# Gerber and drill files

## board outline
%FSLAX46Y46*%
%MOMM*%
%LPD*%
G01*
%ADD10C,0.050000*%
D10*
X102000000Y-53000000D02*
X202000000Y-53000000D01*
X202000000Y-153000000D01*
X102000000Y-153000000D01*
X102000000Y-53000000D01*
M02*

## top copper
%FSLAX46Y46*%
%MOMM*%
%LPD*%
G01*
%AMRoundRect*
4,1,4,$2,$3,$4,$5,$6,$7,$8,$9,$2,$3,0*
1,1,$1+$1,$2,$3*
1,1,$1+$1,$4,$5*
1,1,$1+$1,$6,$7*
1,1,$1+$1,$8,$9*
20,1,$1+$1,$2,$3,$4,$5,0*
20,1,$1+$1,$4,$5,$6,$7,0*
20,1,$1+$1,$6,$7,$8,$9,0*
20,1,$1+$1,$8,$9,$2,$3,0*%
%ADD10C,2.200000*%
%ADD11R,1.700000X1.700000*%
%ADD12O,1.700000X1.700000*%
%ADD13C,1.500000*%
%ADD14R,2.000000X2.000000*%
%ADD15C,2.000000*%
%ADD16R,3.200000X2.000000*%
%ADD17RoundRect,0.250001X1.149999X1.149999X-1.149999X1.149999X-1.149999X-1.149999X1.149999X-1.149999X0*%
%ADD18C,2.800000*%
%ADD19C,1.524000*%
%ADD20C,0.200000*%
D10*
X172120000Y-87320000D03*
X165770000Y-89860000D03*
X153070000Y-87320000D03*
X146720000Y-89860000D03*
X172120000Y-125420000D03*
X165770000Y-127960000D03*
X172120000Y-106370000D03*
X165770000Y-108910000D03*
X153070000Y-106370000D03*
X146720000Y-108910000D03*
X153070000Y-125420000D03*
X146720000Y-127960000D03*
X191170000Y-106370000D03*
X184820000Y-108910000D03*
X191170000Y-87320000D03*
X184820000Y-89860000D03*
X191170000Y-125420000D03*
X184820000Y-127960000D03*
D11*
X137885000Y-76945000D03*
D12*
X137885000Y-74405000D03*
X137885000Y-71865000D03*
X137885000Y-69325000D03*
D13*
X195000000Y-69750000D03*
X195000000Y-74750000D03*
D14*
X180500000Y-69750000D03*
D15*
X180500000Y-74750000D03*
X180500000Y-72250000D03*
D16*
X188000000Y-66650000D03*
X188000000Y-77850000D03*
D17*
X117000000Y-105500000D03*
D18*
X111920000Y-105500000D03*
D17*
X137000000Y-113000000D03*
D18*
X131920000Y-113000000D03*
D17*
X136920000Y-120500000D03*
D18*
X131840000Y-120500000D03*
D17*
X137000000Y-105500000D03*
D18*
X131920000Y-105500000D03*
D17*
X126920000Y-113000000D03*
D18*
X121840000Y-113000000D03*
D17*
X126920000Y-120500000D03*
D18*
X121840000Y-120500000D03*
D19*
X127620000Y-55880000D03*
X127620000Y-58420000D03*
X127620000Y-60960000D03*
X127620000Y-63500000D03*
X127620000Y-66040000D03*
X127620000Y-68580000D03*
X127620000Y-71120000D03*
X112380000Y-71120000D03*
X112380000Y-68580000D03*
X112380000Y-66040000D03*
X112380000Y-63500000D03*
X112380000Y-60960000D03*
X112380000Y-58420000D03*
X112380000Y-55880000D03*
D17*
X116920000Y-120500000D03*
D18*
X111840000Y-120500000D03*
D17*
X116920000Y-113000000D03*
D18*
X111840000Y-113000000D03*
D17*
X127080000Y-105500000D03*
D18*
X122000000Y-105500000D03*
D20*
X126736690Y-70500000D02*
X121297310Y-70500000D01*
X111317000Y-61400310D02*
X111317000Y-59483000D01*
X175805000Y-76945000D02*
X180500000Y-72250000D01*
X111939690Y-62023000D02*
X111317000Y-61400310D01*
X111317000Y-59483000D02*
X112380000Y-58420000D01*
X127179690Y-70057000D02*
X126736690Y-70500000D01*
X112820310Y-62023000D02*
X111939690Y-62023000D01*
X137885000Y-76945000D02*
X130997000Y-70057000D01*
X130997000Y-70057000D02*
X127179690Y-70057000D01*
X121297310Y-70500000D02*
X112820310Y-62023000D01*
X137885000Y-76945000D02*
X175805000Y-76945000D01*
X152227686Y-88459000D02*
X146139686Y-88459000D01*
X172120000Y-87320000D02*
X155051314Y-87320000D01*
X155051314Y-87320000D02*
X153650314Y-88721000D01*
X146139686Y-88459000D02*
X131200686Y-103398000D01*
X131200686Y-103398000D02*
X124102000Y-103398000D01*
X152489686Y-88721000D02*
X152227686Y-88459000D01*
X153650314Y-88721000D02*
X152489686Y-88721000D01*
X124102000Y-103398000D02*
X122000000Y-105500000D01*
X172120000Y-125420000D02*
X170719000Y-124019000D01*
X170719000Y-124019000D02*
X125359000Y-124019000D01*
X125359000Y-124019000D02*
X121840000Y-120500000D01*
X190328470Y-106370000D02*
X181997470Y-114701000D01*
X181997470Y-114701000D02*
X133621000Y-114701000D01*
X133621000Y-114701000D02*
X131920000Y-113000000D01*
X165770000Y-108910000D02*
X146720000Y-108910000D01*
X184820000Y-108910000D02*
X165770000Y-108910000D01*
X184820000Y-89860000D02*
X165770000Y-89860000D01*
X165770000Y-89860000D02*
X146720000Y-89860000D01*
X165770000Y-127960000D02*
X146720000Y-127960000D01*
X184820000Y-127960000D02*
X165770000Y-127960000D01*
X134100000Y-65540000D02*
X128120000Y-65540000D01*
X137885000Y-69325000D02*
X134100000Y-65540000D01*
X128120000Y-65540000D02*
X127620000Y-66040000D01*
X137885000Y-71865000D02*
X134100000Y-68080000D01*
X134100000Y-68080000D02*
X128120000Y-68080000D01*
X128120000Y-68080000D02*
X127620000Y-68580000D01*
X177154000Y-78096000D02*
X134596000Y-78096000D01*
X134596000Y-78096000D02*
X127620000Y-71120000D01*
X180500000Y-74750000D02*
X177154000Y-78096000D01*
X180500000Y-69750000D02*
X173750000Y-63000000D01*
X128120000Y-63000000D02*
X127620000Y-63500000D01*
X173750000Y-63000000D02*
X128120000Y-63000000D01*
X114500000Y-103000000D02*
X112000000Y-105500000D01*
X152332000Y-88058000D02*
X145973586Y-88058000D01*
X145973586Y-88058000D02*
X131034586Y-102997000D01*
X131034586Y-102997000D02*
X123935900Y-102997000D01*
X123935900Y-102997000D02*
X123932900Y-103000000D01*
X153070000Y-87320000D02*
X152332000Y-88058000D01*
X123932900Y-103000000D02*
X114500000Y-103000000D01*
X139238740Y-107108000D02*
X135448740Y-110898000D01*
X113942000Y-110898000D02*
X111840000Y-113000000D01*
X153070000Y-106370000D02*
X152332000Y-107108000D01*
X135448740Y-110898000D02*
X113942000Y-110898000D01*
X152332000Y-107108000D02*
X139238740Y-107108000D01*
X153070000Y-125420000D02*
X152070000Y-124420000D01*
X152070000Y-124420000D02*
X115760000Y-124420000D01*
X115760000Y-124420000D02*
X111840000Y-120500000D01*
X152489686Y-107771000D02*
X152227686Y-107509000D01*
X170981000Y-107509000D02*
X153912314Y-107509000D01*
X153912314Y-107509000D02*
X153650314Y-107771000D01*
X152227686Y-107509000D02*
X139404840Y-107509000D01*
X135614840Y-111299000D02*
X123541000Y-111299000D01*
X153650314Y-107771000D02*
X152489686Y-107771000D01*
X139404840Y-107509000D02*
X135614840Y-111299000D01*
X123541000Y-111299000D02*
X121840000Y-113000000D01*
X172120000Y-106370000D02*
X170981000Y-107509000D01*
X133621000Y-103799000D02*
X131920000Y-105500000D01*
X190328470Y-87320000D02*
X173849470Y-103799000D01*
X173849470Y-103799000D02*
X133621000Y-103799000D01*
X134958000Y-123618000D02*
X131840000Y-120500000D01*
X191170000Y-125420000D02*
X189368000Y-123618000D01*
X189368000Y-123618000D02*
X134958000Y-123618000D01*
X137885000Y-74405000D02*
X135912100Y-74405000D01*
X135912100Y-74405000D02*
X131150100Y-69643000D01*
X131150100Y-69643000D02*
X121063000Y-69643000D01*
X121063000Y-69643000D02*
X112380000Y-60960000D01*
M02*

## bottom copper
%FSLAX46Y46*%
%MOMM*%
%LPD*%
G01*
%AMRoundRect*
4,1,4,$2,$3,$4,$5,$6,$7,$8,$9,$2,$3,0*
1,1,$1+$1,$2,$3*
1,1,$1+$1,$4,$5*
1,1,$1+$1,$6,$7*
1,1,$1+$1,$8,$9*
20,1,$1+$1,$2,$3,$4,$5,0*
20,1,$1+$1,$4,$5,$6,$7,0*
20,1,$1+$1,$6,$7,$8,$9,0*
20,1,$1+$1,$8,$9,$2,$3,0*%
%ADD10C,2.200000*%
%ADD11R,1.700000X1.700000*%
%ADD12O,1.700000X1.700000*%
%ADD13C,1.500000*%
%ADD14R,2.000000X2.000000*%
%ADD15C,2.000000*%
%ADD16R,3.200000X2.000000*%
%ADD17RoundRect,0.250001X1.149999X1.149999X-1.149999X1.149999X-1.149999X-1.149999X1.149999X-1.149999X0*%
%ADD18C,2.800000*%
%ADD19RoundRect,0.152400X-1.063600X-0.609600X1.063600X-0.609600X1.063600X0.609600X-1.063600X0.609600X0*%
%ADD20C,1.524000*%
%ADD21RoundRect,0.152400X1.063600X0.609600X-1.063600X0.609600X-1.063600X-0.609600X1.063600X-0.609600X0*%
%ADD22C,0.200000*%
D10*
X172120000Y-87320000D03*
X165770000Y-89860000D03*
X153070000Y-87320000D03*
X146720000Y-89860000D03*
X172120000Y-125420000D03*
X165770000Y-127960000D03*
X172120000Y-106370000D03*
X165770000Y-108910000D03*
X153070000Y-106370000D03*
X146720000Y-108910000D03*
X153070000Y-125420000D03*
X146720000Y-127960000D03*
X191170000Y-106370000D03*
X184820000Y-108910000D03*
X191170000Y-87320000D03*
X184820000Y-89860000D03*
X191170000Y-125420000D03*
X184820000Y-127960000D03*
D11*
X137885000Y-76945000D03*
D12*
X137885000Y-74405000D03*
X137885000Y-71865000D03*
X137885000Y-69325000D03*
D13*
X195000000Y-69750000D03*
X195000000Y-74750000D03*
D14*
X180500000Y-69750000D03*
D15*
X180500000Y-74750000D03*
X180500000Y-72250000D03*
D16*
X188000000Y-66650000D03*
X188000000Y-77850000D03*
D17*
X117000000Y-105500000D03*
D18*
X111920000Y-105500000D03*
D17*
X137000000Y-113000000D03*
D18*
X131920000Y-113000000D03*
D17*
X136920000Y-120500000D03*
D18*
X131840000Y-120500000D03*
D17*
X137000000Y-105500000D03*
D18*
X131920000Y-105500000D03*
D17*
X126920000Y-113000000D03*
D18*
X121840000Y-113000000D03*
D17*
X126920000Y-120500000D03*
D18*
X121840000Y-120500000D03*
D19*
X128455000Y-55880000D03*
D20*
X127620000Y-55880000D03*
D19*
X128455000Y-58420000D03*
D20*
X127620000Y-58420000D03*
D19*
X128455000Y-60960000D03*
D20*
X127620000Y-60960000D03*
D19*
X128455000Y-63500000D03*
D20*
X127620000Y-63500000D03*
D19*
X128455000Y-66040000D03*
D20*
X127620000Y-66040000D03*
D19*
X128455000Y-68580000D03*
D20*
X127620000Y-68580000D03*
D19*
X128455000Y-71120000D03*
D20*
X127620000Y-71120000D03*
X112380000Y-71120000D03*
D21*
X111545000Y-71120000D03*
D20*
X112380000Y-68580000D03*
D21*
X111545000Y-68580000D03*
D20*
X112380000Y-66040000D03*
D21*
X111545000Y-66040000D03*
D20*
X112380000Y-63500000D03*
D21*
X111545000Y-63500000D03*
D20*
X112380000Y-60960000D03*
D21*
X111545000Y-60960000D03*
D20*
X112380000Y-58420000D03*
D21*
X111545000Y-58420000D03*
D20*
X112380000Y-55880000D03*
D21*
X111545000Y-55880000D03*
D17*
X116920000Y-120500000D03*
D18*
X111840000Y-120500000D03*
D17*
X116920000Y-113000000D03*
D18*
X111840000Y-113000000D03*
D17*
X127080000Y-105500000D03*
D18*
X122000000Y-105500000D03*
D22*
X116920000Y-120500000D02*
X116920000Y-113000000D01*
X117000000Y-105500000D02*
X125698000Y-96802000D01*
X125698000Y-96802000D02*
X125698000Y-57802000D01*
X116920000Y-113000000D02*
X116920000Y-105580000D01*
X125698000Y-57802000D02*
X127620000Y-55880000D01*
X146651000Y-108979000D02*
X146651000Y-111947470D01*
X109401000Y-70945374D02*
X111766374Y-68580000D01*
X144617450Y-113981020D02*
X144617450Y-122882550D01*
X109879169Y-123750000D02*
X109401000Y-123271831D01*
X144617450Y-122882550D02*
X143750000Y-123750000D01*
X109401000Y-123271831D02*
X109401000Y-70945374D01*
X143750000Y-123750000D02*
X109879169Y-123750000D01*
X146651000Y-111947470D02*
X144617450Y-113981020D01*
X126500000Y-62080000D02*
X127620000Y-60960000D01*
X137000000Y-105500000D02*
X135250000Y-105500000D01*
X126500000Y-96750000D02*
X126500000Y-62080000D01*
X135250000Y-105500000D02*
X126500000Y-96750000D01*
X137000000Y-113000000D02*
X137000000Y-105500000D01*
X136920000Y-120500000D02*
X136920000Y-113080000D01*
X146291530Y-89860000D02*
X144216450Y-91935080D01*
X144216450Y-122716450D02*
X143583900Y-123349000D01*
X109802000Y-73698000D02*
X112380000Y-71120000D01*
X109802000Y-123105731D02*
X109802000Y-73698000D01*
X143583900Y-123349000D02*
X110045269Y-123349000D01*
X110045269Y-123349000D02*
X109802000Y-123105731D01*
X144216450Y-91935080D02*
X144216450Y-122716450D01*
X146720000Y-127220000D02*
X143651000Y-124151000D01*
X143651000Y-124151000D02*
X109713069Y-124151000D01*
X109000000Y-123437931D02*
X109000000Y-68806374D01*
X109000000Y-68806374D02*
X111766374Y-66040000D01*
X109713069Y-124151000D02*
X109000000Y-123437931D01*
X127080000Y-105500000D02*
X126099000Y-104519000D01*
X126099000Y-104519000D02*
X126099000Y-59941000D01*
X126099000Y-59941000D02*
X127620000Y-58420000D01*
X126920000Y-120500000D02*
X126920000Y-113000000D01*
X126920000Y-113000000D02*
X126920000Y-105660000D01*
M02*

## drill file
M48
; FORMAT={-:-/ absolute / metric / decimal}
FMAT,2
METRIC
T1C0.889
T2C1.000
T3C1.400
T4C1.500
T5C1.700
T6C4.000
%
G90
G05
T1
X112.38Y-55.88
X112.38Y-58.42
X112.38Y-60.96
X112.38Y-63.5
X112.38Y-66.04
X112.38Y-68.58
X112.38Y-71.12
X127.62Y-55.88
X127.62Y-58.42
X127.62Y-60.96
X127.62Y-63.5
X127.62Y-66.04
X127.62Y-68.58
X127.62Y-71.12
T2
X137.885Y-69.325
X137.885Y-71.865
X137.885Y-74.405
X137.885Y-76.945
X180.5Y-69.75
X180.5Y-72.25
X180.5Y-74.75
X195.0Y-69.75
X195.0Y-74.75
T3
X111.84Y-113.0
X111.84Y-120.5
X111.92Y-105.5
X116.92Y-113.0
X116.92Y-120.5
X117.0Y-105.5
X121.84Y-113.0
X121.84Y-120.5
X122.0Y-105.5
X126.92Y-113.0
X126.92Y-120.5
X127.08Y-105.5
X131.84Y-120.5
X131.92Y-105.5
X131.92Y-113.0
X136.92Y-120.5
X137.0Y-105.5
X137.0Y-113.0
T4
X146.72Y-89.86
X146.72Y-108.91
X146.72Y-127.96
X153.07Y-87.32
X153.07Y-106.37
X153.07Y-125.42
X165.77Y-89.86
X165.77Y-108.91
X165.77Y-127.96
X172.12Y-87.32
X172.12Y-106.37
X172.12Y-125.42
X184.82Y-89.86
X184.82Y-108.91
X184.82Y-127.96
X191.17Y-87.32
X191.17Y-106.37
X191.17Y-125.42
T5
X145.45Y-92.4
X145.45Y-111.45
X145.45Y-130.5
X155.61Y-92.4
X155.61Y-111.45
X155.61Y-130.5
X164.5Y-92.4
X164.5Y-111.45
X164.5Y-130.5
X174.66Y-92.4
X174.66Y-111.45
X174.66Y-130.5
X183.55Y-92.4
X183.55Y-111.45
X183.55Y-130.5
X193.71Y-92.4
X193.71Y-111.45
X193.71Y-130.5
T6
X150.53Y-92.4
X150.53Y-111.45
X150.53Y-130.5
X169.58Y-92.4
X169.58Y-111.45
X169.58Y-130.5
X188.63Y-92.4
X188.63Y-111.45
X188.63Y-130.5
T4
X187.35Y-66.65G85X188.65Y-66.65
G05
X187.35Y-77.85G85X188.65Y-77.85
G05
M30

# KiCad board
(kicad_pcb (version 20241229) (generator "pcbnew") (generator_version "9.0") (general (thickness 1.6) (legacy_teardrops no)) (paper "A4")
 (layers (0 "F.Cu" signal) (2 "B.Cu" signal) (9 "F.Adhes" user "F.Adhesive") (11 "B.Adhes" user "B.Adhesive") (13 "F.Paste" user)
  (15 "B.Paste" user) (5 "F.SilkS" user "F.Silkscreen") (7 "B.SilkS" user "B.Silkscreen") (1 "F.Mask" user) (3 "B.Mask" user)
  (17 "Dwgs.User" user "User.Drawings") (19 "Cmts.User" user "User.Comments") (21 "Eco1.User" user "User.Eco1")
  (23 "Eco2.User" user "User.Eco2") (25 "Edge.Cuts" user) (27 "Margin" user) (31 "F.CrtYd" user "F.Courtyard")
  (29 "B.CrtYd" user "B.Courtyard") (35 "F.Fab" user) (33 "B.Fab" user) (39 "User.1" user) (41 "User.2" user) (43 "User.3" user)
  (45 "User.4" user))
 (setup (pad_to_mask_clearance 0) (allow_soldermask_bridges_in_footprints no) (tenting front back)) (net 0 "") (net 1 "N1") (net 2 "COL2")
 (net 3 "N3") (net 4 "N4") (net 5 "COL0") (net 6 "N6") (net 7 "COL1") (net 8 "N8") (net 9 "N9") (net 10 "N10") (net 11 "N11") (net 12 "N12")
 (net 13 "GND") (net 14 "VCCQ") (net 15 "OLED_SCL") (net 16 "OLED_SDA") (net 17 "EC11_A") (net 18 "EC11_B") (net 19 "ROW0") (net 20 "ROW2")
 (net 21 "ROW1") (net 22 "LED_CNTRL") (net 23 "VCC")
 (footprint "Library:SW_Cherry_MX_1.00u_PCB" (layer "F.Cu") (at 172.12 87.32)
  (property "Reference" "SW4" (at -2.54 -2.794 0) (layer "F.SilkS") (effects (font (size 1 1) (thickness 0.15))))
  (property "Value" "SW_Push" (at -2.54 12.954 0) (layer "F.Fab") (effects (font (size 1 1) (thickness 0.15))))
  (pad "" np_thru_hole circle (at -7.62 5.08) (size 1.7 1.7) (drill 1.7) (layers "*.Cu" "*.Mask"))
  (pad "" np_thru_hole circle (at -2.54 5.08) (size 4 4) (drill 4) (layers "*.Cu" "*.Mask"))
  (pad "" np_thru_hole circle (at 2.54 5.08) (size 1.7 1.7) (drill 1.7) (layers "*.Cu" "*.Mask"))
  (pad "1" thru_hole circle (at 0 0) (size 2.2 2.2) (drill 1.5) (layers "*.Cu" "*.Mask") (remove_unused_layers no) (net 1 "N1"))
  (pad "2" thru_hole circle (at -6.35 2.54) (size 2.2 2.2) (drill 1.5) (layers "*.Cu" "*.Mask") (remove_unused_layers no) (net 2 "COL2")))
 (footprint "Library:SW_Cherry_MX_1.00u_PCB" (layer "F.Cu") (at 153.07 87.32)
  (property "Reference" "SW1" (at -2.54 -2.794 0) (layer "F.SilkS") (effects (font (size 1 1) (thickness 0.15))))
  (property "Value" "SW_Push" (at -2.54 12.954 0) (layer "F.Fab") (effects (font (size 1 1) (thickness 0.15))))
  (pad "" np_thru_hole circle (at -7.62 5.08) (size 1.7 1.7) (drill 1.7) (layers "*.Cu" "*.Mask"))
  (pad "" np_thru_hole circle (at -2.54 5.08) (size 4 4) (drill 4) (layers "*.Cu" "*.Mask"))
  (pad "" np_thru_hole circle (at 2.54 5.08) (size 1.7 1.7) (drill 1.7) (layers "*.Cu" "*.Mask"))
  (pad "1" thru_hole circle (at 0 0) (size 2.2 2.2) (drill 1.5) (layers "*.Cu" "*.Mask") (remove_unused_layers no) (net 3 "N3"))
  (pad "2" thru_hole circle (at -6.35 2.54) (size 2.2 2.2) (drill 1.5) (layers "*.Cu" "*.Mask") (remove_unused_layers no) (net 2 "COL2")))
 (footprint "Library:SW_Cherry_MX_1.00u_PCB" (layer "F.Cu") (at 172.12 125.42)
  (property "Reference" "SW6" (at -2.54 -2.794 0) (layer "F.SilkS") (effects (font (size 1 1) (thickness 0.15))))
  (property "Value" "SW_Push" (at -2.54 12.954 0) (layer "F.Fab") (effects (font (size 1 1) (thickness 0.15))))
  (pad "" np_thru_hole circle (at -7.62 5.08) (size 1.7 1.7) (drill 1.7) (layers "*.Cu" "*.Mask"))
  (pad "" np_thru_hole circle (at -2.54 5.08) (size 4 4) (drill 4) (layers "*.Cu" "*.Mask"))
  (pad "" np_thru_hole circle (at 2.54 5.08) (size 1.7 1.7) (drill 1.7) (layers "*.Cu" "*.Mask"))
  (pad "1" thru_hole circle (at 0 0) (size 2.2 2.2) (drill 1.5) (layers "*.Cu" "*.Mask") (remove_unused_layers no) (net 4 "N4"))
  (pad "2" thru_hole circle (at -6.35 2.54) (size 2.2 2.2) (drill 1.5) (layers "*.Cu" "*.Mask") (remove_unused_layers no) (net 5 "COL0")))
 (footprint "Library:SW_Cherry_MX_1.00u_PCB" (layer "F.Cu") (at 172.12 106.37)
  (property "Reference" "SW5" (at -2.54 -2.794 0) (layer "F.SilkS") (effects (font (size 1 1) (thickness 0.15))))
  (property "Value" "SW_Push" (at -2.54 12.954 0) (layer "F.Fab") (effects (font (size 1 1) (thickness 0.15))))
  (pad "" np_thru_hole circle (at -7.62 5.08) (size 1.7 1.7) (drill 1.7) (layers "*.Cu" "*.Mask"))
  (pad "" np_thru_hole circle (at -2.54 5.08) (size 4 4) (drill 4) (layers "*.Cu" "*.Mask"))
  (pad "" np_thru_hole circle (at 2.54 5.08) (size 1.7 1.7) (drill 1.7) (layers "*.Cu" "*.Mask"))
  (pad "1" thru_hole circle (at 0 0) (size 2.2 2.2) (drill 1.5) (layers "*.Cu" "*.Mask") (remove_unused_layers no) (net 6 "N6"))
  (pad "2" thru_hole circle (at -6.35 2.54) (size 2.2 2.2) (drill 1.5) (layers "*.Cu" "*.Mask") (remove_unused_layers no) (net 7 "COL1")))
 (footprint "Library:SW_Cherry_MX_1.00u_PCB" (layer "F.Cu") (at 153.07 106.37)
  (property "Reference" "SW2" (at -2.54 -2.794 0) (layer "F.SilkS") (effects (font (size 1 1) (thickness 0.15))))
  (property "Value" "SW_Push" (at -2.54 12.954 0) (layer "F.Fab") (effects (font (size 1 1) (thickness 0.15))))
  (pad "" np_thru_hole circle (at -7.62 5.08) (size 1.7 1.7) (drill 1.7) (layers "*.Cu" "*.Mask"))
  (pad "" np_thru_hole circle (at -2.54 5.08) (size 4 4) (drill 4) (layers "*.Cu" "*.Mask"))
  (pad "" np_thru_hole circle (at 2.54 5.08) (size 1.7 1.7) (drill 1.7) (layers "*.Cu" "*.Mask"))
  (pad "1" thru_hole circle (at 0 0) (size 2.2 2.2) (drill 1.5) (layers "*.Cu" "*.Mask") (remove_unused_layers no) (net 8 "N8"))
  (pad "2" thru_hole circle (at -6.35 2.54) (size 2.2 2.2) (drill 1.5) (layers "*.Cu" "*.Mask") (remove_unused_layers no) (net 7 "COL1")))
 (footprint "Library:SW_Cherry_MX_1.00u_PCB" (layer "F.Cu") (at 153.07 125.42)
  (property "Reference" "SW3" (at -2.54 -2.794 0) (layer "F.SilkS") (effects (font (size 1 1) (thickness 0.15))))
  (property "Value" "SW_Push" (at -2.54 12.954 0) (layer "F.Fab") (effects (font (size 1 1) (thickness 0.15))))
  (pad "" np_thru_hole circle (at -7.62 5.08) (size 1.7 1.7) (drill 1.7) (layers "*.Cu" "*.Mask"))
  (pad "" np_thru_hole circle (at -2.54 5.08) (size 4 4) (drill 4) (layers "*.Cu" "*.Mask"))
  (pad "" np_thru_hole circle (at 2.54 5.08) (size 1.7 1.7) (drill 1.7) (layers "*.Cu" "*.Mask"))
  (pad "1" thru_hole circle (at 0 0) (size 2.2 2.2) (drill 1.5) (layers "*.Cu" "*.Mask") (remove_unused_layers no) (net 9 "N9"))
  (pad "2" thru_hole circle (at -6.35 2.54) (size 2.2 2.2) (drill 1.5) (layers "*.Cu" "*.Mask") (remove_unused_layers no) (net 5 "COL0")))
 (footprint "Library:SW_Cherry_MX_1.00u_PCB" (layer "F.Cu") (at 191.17 106.37)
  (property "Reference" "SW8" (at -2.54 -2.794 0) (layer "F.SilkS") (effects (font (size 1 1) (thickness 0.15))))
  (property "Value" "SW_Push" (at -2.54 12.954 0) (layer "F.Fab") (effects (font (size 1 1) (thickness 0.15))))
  (pad "" np_thru_hole circle (at -7.62 5.08) (size 1.7 1.7) (drill 1.7) (layers "*.Cu" "*.Mask"))
  (pad "" np_thru_hole circle (at -2.54 5.08) (size 4 4) (drill 4) (layers "*.Cu" "*.Mask"))
  (pad "" np_thru_hole circle (at 2.54 5.08) (size 1.7 1.7) (drill 1.7) (layers "*.Cu" "*.Mask"))
  (pad "1" thru_hole circle (at 0 0) (size 2.2 2.2) (drill 1.5) (layers "*.Cu" "*.Mask") (remove_unused_layers no) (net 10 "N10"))
  (pad "2" thru_hole circle (at -6.35 2.54) (size 2.2 2.2) (drill 1.5) (layers "*.Cu" "*.Mask") (remove_unused_layers no) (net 7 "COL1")))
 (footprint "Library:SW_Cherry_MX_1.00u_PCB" (layer "F.Cu") (at 191.17 87.32)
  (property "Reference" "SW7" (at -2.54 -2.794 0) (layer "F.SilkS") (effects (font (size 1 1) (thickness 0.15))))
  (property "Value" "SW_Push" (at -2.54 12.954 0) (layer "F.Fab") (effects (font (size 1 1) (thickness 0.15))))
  (pad "" np_thru_hole circle (at -7.62 5.08) (size 1.7 1.7) (drill 1.7) (layers "*.Cu" "*.Mask"))
  (pad "" np_thru_hole circle (at -2.54 5.08) (size 4 4) (drill 4) (layers "*.Cu" "*.Mask"))
  (pad "" np_thru_hole circle (at 2.54 5.08) (size 1.7 1.7) (drill 1.7) (layers "*.Cu" "*.Mask"))
  (pad "1" thru_hole circle (at 0 0) (size 2.2 2.2) (drill 1.5) (layers "*.Cu" "*.Mask") (remove_unused_layers no) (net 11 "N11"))
  (pad "2" thru_hole circle (at -6.35 2.54) (size 2.2 2.2) (drill 1.5) (layers "*.Cu" "*.Mask") (remove_unused_layers no) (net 2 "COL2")))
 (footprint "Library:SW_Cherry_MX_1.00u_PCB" (layer "F.Cu") (at 191.17 125.42)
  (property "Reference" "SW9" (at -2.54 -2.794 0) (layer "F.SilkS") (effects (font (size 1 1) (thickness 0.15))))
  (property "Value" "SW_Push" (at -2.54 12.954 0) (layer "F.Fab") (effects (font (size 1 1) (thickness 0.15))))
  (pad "" np_thru_hole circle (at -7.62 5.08) (size 1.7 1.7) (drill 1.7) (layers "*.Cu" "*.Mask"))
  (pad "" np_thru_hole circle (at -2.54 5.08) (size 4 4) (drill 4) (layers "*.Cu" "*.Mask"))
  (pad "" np_thru_hole circle (at 2.54 5.08) (size 1.7 1.7) (drill 1.7) (layers "*.Cu" "*.Mask"))
  (pad "1" thru_hole circle (at 0 0) (size 2.2 2.2) (drill 1.5) (layers "*.Cu" "*.Mask") (remove_unused_layers no) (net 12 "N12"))
  (pad "2" thru_hole circle (at -6.35 2.54) (size 2.2 2.2) (drill 1.5) (layers "*.Cu" "*.Mask") (remove_unused_layers no) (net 5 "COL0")))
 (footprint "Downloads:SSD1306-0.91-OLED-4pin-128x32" (layer "F.Cu") (at 174.385 79.135 180)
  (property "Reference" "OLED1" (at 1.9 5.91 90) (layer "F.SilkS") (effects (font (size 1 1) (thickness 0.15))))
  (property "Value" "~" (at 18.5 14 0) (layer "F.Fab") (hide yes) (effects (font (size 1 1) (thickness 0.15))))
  (pad "1" thru_hole rect (at 36.5 2.19 180) (size 1.7 1.7) (drill 1) (layers "*.Cu" "*.Mask") (remove_unused_layers no) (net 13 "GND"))
  (pad "2" thru_hole oval (at 36.5 4.73 180) (size 1.7 1.7) (drill 1) (layers "*.Cu" "*.Mask") (remove_unused_layers no) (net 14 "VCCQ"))
  (pad "3" thru_hole oval (at 36.5 7.27 180) (size 1.7 1.7) (drill 1) (layers "*.Cu" "*.Mask") (remove_unused_layers no) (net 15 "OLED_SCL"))
  (pad "4" thru_hole oval (at 36.5 9.81 180) (size 1.7 1.7) (drill 1) (layers "*.Cu" "*.Mask") (remove_unused_layers no) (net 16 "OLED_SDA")))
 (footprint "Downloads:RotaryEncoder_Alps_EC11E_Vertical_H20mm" (layer "F.Cu") (at 180.5 69.75)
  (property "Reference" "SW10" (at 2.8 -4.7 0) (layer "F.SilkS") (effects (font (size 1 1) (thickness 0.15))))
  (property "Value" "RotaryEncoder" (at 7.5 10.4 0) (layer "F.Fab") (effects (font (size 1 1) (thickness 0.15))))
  (pad "" thru_hole circle (at 14.5 0) (size 1.5 1.5) (drill 1) (layers "*.Cu" "*.Mask") (remove_unused_layers no))
  (pad "" thru_hole circle (at 14.5 5) (size 1.5 1.5) (drill 1) (layers "*.Cu" "*.Mask") (remove_unused_layers no))
  (pad "A" thru_hole rect (at 0 0) (size 2 2) (drill 1) (layers "*.Cu" "*.Mask") (remove_unused_layers no) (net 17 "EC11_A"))
  (pad "B" thru_hole circle (at 0 5) (size 2 2) (drill 1) (layers "*.Cu" "*.Mask") (remove_unused_layers no) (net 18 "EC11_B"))
  (pad "C" thru_hole circle (at 0 2.5) (size 2 2) (drill 1) (layers "*.Cu" "*.Mask") (remove_unused_layers no) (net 13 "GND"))
  (pad "MP" thru_hole rect (at 7.5 -3.1) (size 3.2 2) (drill oval 2.8 1.5) (layers "*.Cu" "*.Mask") (remove_unused_layers no))
  (pad "MP" thru_hole rect (at 7.5 8.1) (size 3.2 2) (drill oval 2.8 1.5) (layers "*.Cu" "*.Mask") (remove_unused_layers no)))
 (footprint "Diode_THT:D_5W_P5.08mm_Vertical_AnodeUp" (layer "B.Cu") (at 117 105.5 180)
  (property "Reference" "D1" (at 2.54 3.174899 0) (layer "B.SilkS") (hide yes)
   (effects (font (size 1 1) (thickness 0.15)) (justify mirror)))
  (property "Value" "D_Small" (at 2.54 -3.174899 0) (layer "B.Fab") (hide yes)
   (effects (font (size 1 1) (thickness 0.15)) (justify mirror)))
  (pad "1" thru_hole roundrect (at 0 0 180) (size 2.8 2.8) (drill 1.4) (layers "*.Cu" "*.Mask") (remove_unused_layers no)
   (roundrect_rratio 0.089286) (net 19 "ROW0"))
  (pad "2" thru_hole circle (at 5.08 0 180) (size 2.8 2.8) (drill 1.4) (layers "*.Cu" "*.Mask") (remove_unused_layers no) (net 3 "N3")))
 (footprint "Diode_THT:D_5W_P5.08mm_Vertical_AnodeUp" (layer "B.Cu") (at 137 113 180)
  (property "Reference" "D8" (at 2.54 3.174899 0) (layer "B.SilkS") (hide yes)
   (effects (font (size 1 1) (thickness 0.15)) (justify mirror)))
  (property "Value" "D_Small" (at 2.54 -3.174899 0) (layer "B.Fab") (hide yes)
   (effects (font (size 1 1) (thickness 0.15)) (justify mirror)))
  (pad "1" thru_hole roundrect (at 0 0 180) (size 2.8 2.8) (drill 1.4) (layers "*.Cu" "*.Mask") (remove_unused_layers no)
   (roundrect_rratio 0.089286) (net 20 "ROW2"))
  (pad "2" thru_hole circle (at 5.08 0 180) (size 2.8 2.8) (drill 1.4) (layers "*.Cu" "*.Mask") (remove_unused_layers no) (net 10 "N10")))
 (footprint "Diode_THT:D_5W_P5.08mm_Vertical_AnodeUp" (layer "B.Cu") (at 136.92 120.5 180)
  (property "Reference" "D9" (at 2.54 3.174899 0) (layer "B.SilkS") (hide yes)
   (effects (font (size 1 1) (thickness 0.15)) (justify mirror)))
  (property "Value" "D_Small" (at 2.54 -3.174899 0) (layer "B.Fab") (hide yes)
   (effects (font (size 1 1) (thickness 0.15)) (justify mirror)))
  (pad "1" thru_hole roundrect (at 0 0 180) (size 2.8 2.8) (drill 1.4) (layers "*.Cu" "*.Mask") (remove_unused_layers no)
   (roundrect_rratio 0.089286) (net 20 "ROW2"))
  (pad "2" thru_hole circle (at 5.08 0 180) (size 2.8 2.8) (drill 1.4) (layers "*.Cu" "*.Mask") (remove_unused_layers no) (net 12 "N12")))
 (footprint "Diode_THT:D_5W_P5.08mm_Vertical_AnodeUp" (layer "B.Cu") (at 137 105.5 180)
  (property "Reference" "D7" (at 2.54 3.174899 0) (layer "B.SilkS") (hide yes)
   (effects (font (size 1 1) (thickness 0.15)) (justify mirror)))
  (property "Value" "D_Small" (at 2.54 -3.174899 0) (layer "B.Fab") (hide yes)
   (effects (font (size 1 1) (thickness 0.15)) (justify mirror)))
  (pad "1" thru_hole roundrect (at 0 0 180) (size 2.8 2.8) (drill 1.4) (layers "*.Cu" "*.Mask") (remove_unused_layers no)
   (roundrect_rratio 0.089286) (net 20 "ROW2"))
  (pad "2" thru_hole circle (at 5.08 0 180) (size 2.8 2.8) (drill 1.4) (layers "*.Cu" "*.Mask") (remove_unused_layers no) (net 11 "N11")))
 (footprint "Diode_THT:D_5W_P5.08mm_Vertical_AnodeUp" (layer "B.Cu") (at 126.92 113 180)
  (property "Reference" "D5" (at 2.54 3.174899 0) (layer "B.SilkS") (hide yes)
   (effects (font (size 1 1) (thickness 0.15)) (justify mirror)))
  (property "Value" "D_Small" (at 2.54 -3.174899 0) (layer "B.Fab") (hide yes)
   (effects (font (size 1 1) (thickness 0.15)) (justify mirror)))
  (pad "1" thru_hole roundrect (at 0 0 180) (size 2.8 2.8) (drill 1.4) (layers "*.Cu" "*.Mask") (remove_unused_layers no)
   (roundrect_rratio 0.089286) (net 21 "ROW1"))
  (pad "2" thru_hole circle (at 5.08 0 180) (size 2.8 2.8) (drill 1.4) (layers "*.Cu" "*.Mask") (remove_unused_layers no) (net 6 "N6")))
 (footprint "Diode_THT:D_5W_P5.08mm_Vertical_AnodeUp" (layer "B.Cu") (at 126.92 120.5 180)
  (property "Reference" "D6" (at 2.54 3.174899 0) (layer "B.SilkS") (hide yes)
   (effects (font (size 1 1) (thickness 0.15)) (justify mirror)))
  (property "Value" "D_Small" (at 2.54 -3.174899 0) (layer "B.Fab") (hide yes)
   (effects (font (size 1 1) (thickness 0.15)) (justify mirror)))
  (pad "1" thru_hole roundrect (at 0 0 180) (size 2.8 2.8) (drill 1.4) (layers "*.Cu" "*.Mask") (remove_unused_layers no)
   (roundrect_rratio 0.089286) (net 21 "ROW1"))
  (pad "2" thru_hole circle (at 5.08 0 180) (size 2.8 2.8) (drill 1.4) (layers "*.Cu" "*.Mask") (remove_unused_layers no) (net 4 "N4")))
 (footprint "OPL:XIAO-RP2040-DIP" (layer "B.Cu") (at 120 63.5 180)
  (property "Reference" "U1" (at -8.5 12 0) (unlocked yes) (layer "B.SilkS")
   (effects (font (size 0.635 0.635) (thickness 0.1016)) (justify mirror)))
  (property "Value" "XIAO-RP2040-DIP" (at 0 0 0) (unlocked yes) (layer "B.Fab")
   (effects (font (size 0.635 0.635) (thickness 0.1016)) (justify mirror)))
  (pad "1" smd roundrect (at -8.455 7.62) (size 2.432 1.524) (layers "B.Cu" "B.Mask") (roundrect_rratio 0.1) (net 19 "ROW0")
   (thermal_bridge_angle 45))
  (pad "1" thru_hole circle (at -7.62 7.62) (size 1.524 1.524) (drill 0.889) (layers "*.Cu" "*.Mask") (remove_unused_layers no)
   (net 19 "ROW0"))
  (pad "2" smd roundrect (at -8.455 5.08) (size 2.432 1.524) (layers "B.Cu" "B.Mask") (roundrect_rratio 0.1) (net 21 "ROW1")
   (thermal_bridge_angle 45))
  (pad "2" thru_hole circle (at -7.62 5.08) (size 1.524 1.524) (drill 0.889) (layers "*.Cu" "*.Mask") (remove_unused_layers no)
   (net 21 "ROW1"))
  (pad "3" smd roundrect (at -8.455 2.54) (size 2.432 1.524) (layers "B.Cu" "B.Mask") (roundrect_rratio 0.1) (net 20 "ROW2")
   (thermal_bridge_angle 45))
  (pad "3" thru_hole circle (at -7.62 2.54) (size 1.524 1.524) (drill 0.889) (layers "*.Cu" "*.Mask") (remove_unused_layers no)
   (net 20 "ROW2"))
  (pad "4" smd roundrect (at -8.455 0) (size 2.432 1.524) (layers "B.Cu" "B.Mask") (roundrect_rratio 0.1) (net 17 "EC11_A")
   (thermal_bridge_angle 45))
  (pad "4" thru_hole circle (at -7.62 0) (size 1.524 1.524) (drill 0.889) (layers "*.Cu" "*.Mask") (remove_unused_layers no)
   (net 17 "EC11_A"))
  (pad "5" smd roundrect (at -8.455 -2.54) (size 2.432 1.524) (layers "B.Cu" "B.Mask") (roundrect_rratio 0.1) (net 16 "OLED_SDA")
   (thermal_bridge_angle 45))
  (pad "5" thru_hole circle (at -7.62 -2.54) (size 1.524 1.524) (drill 0.889) (layers "*.Cu" "*.Mask") (remove_unused_layers no)
   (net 16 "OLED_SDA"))
  (pad "6" smd roundrect (at -8.455 -5.08) (size 2.432 1.524) (layers "B.Cu" "B.Mask") (roundrect_rratio 0.1) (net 15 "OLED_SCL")
   (thermal_bridge_angle 45))
  (pad "6" thru_hole circle (at -7.62 -5.08) (size 1.524 1.524) (drill 0.889) (layers "*.Cu" "*.Mask") (remove_unused_layers no)
   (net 15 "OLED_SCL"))
  (pad "7" smd roundrect (at -8.455 -7.62) (size 2.432 1.524) (layers "B.Cu" "B.Mask") (roundrect_rratio 0.1) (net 18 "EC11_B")
   (thermal_bridge_angle 45))
  (pad "7" thru_hole circle (at -7.62 -7.62) (size 1.524 1.524) (drill 0.889) (layers "*.Cu" "*.Mask") (remove_unused_layers no)
   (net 18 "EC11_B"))
  (pad "8" thru_hole circle (at 7.62 -7.62 180) (size 1.524 1.524) (drill 0.889) (layers "*.Cu" "*.Mask") (remove_unused_layers no)
   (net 2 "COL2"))
  (pad "8" smd roundrect (at 8.455 -7.62 180) (size 2.432 1.524) (layers "B.Cu" "B.Mask") (roundrect_rratio 0.1) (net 2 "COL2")
   (thermal_bridge_angle 45))
  (pad "9" thru_hole circle (at 7.62 -5.08 180) (size 1.524 1.524) (drill 0.889) (layers "*.Cu" "*.Mask") (remove_unused_layers no)
   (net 7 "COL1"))
  (pad "9" smd roundrect (at 8.455 -5.08 180) (size 2.432 1.524) (layers "B.Cu" "B.Mask") (roundrect_rratio 0.1) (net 7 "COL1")
   (thermal_bridge_angle 45))
  (pad "10" thru_hole circle (at 7.62 -2.54 180) (size 1.524 1.524) (drill 0.889) (layers "*.Cu" "*.Mask") (remove_unused_layers no)
   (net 5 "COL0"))
  (pad "10" smd roundrect (at 8.455 -2.54 180) (size 2.432 1.524) (layers "B.Cu" "B.Mask") (roundrect_rratio 0.1) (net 5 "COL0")
   (thermal_bridge_angle 45))
  (pad "11" thru_hole circle (at 7.62 0 180) (size 1.524 1.524) (drill 0.889) (layers "*.Cu" "*.Mask") (remove_unused_layers no)
   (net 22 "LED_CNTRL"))
  (pad "11" smd roundrect (at 8.455 0 180) (size 2.432 1.524) (layers "B.Cu" "B.Mask") (roundrect_rratio 0.1) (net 22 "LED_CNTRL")
   (thermal_bridge_angle 45))
  (pad "12" thru_hole circle (at 7.62 2.54 180) (size 1.524 1.524) (drill 0.889) (layers "*.Cu" "*.Mask") (remove_unused_layers no)
   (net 14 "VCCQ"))
  (pad "12" smd roundrect (at 8.455 2.54 180) (size 2.432 1.524) (layers "B.Cu" "B.Mask") (roundrect_rratio 0.1) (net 14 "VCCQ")
   (thermal_bridge_angle 45))
  (pad "13" thru_hole circle (at 7.62 5.08 180) (size 1.524 1.524) (drill 0.889) (layers "*.Cu" "*.Mask") (remove_unused_layers no)
   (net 13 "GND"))
  (pad "13" smd roundrect (at 8.455 5.08 180) (size 2.432 1.524) (layers "B.Cu" "B.Mask") (roundrect_rratio 0.1) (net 13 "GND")
   (thermal_bridge_angle 45))
  (pad "14" thru_hole circle (at 7.62 7.62 180) (size 1.524 1.524) (drill 0.889) (layers "*.Cu" "*.Mask") (remove_unused_layers no)
   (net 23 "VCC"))
  (pad "14" smd roundrect (at 8.455 7.62 180) (size 2.432 1.524) (layers "B.Cu" "B.Mask") (roundrect_rratio 0.1) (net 23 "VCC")
   (thermal_bridge_angle 45)))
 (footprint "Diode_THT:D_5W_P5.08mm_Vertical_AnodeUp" (layer "B.Cu") (at 116.92 120.5 180)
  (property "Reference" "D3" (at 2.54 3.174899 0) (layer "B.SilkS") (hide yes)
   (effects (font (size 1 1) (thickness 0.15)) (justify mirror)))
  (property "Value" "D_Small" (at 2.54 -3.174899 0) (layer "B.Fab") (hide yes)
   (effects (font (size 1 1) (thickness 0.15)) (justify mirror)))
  (pad "1" thru_hole roundrect (at 0 0 180) (size 2.8 2.8) (drill 1.4) (layers "*.Cu" "*.Mask") (remove_unused_layers no)
   (roundrect_rratio 0.089286) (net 19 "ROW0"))
  (pad "2" thru_hole circle (at 5.08 0 180) (size 2.8 2.8) (drill 1.4) (layers "*.Cu" "*.Mask") (remove_unused_layers no) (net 9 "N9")))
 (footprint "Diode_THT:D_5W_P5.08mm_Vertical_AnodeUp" (layer "B.Cu") (at 116.92 113 180)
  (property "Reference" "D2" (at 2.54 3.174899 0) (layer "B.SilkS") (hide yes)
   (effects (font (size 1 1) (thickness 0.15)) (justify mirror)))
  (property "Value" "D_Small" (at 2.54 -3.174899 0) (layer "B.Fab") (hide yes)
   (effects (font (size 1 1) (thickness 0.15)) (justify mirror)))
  (pad "1" thru_hole roundrect (at 0 0 180) (size 2.8 2.8) (drill 1.4) (layers "*.Cu" "*.Mask") (remove_unused_layers no)
   (roundrect_rratio 0.089286) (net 19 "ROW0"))
  (pad "2" thru_hole circle (at 5.08 0 180) (size 2.8 2.8) (drill 1.4) (layers "*.Cu" "*.Mask") (remove_unused_layers no) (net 8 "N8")))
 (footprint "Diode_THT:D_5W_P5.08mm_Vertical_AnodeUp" (layer "B.Cu") (at 127.08 105.5 180)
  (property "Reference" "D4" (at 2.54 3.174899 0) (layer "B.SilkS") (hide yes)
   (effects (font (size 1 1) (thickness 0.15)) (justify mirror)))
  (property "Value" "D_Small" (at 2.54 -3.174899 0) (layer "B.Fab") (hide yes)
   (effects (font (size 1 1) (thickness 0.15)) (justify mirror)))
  (pad "1" thru_hole roundrect (at 0 0 180) (size 2.8 2.8) (drill 1.4) (layers "*.Cu" "*.Mask") (remove_unused_layers no)
   (roundrect_rratio 0.089286) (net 21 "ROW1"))
  (pad "2" thru_hole circle (at 5.08 0 180) (size 2.8 2.8) (drill 1.4) (layers "*.Cu" "*.Mask") (remove_unused_layers no) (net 1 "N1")))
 (gr_rect (start 102 53) (end 202 153) (stroke (width 0.05) (type default)) (fill no) (layer "Edge.Cuts"))
 (segment (start 126.73669 70.5) (end 121.29731 70.5) (width 0.2) (layer "F.Cu") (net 13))
 (segment (start 111.317 61.40031) (end 111.317 59.483) (width 0.2) (layer "F.Cu") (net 13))
 (segment (start 175.805 76.945) (end 180.5 72.25) (width 0.2) (layer "F.Cu") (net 13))
 (segment (start 111.93969 62.023) (end 111.317 61.40031) (width 0.2) (layer "F.Cu") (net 13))
 (segment (start 111.317 59.483) (end 112.38 58.42) (width 0.2) (layer "F.Cu") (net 13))
 (segment (start 127.17969 70.057) (end 126.73669 70.5) (width 0.2) (layer "F.Cu") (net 13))
 (segment (start 112.82031 62.023) (end 111.93969 62.023) (width 0.2) (layer "F.Cu") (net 13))
 (segment (start 137.885 76.945) (end 130.997 70.057) (width 0.2) (layer "F.Cu") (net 13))
 (segment (start 130.997 70.057) (end 127.17969 70.057) (width 0.2) (layer "F.Cu") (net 13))
 (segment (start 121.29731 70.5) (end 112.82031 62.023) (width 0.2) (layer "F.Cu") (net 13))
 (segment (start 137.885 76.945) (end 175.805 76.945) (width 0.2) (layer "F.Cu") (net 13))
 (segment (start 116.92 120.5) (end 116.92 113) (width 0.2) (layer "B.Cu") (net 19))
 (segment (start 117 105.5) (end 125.698 96.802) (width 0.2) (layer "B.Cu") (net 19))
 (segment (start 125.698 96.802) (end 125.698 57.802) (width 0.2) (layer "B.Cu") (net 19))
 (segment (start 116.92 113) (end 116.92 105.58) (width 0.2) (layer "B.Cu") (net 19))
 (segment (start 125.698 57.802) (end 127.62 55.88) (width 0.2) (layer "B.Cu") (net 19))
 (segment (start 152.227686 88.459) (end 146.139686 88.459) (width 0.2) (layer "F.Cu") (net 1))
 (segment (start 172.12 87.32) (end 155.051314 87.32) (width 0.2) (layer "F.Cu") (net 1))
 (segment (start 155.051314 87.32) (end 153.650314 88.721) (width 0.2) (layer "F.Cu") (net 1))
 (segment (start 146.139686 88.459) (end 131.200686 103.398) (width 0.2) (layer "F.Cu") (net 1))
 (segment (start 131.200686 103.398) (end 124.102 103.398) (width 0.2) (layer "F.Cu") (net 1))
 (segment (start 152.489686 88.721) (end 152.227686 88.459) (width 0.2) (layer "F.Cu") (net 1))
 (segment (start 153.650314 88.721) (end 152.489686 88.721) (width 0.2) (layer "F.Cu") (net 1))
 (segment (start 124.102 103.398) (end 122 105.5) (width 0.2) (layer "F.Cu") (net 1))
 (segment (start 172.12 125.42) (end 170.719 124.019) (width 0.2) (layer "F.Cu") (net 4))
 (segment (start 170.719 124.019) (end 125.359 124.019) (width 0.2) (layer "F.Cu") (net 4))
 (segment (start 125.359 124.019) (end 121.84 120.5) (width 0.2) (layer "F.Cu") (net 4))
 (segment (start 190.32847 106.37) (end 181.99747 114.701) (width 0.2) (layer "F.Cu") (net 10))
 (segment (start 181.99747 114.701) (end 133.621 114.701) (width 0.2) (layer "F.Cu") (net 10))
 (segment (start 133.621 114.701) (end 131.92 113) (width 0.2) (layer "F.Cu") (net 10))
 (segment (start 165.77 108.91) (end 146.72 108.91) (width 0.2) (layer "F.Cu") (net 7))
 (segment (start 184.82 108.91) (end 165.77 108.91) (width 0.2) (layer "F.Cu") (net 7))
 (segment (start 146.651 108.979) (end 146.651 111.94747) (width 0.2) (layer "B.Cu") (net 7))
 (segment (start 109.401 70.945374) (end 111.766374 68.58) (width 0.2) (layer "B.Cu") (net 7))
 (segment (start 144.61745 113.98102) (end 144.61745 122.88255) (width 0.2) (layer "B.Cu") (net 7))
 (segment (start 109.879169 123.75) (end 109.401 123.271831) (width 0.2) (layer "B.Cu") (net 7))
 (segment (start 144.61745 122.88255) (end 143.75 123.75) (width 0.2) (layer "B.Cu") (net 7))
 (segment (start 109.401 123.271831) (end 109.401 70.945374) (width 0.2) (layer "B.Cu") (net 7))
 (segment (start 143.75 123.75) (end 109.879169 123.75) (width 0.2) (layer "B.Cu") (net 7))
 (segment (start 146.651 111.94747) (end 144.61745 113.98102) (width 0.2) (layer "B.Cu") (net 7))
 (segment (start 126.5 62.08) (end 127.62 60.96) (width 0.2) (layer "B.Cu") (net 20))
 (segment (start 137 105.5) (end 135.25 105.5) (width 0.2) (layer "B.Cu") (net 20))
 (segment (start 126.5 96.75) (end 126.5 62.08) (width 0.2) (layer "B.Cu") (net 20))
 (segment (start 135.25 105.5) (end 126.5 96.75) (width 0.2) (layer "B.Cu") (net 20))
 (segment (start 137 113) (end 137 105.5) (width 0.2) (layer "B.Cu") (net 20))
 (segment (start 136.92 120.5) (end 136.92 113.08) (width 0.2) (layer "B.Cu") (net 20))
 (segment (start 184.82 89.86) (end 165.77 89.86) (width 0.2) (layer "F.Cu") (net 2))
 (segment (start 165.77 89.86) (end 146.72 89.86) (width 0.2) (layer "F.Cu") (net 2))
 (segment (start 146.29153 89.86) (end 144.21645 91.93508) (width 0.2) (layer "B.Cu") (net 2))
 (segment (start 144.21645 122.71645) (end 143.5839 123.349) (width 0.2) (layer "B.Cu") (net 2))
 (segment (start 109.802 73.698) (end 112.38 71.12) (width 0.2) (layer "B.Cu") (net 2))
 (segment (start 109.802 123.105731) (end 109.802 73.698) (width 0.2) (layer "B.Cu") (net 2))
 (segment (start 143.5839 123.349) (end 110.045269 123.349) (width 0.2) (layer "B.Cu") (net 2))
 (segment (start 110.045269 123.349) (end 109.802 123.105731) (width 0.2) (layer "B.Cu") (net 2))
 (segment (start 144.21645 91.93508) (end 144.21645 122.71645) (width 0.2) (layer "B.Cu") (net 2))
 (segment (start 165.77 127.96) (end 146.72 127.96) (width 0.2) (layer "F.Cu") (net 5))
 (segment (start 184.82 127.96) (end 165.77 127.96) (width 0.2) (layer "F.Cu") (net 5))
 (segment (start 146.72 127.22) (end 143.651 124.151) (width 0.2) (layer "B.Cu") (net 5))
 (segment (start 143.651 124.151) (end 109.713069 124.151) (width 0.2) (layer "B.Cu") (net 5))
 (segment (start 109 123.437931) (end 109 68.806374) (width 0.2) (layer "B.Cu") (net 5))
 (segment (start 109 68.806374) (end 111.766374 66.04) (width 0.2) (layer "B.Cu") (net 5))
 (segment (start 109.713069 124.151) (end 109 123.437931) (width 0.2) (layer "B.Cu") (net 5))
 (segment (start 127.08 105.5) (end 126.099 104.519) (width 0.2) (layer "B.Cu") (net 21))
 (segment (start 126.099 104.519) (end 126.099 59.941) (width 0.2) (layer "B.Cu") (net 21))
 (segment (start 126.099 59.941) (end 127.62 58.42) (width 0.2) (layer "B.Cu") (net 21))
 (segment (start 126.92 120.5) (end 126.92 113) (width 0.2) (layer "B.Cu") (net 21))
 (segment (start 126.92 113) (end 126.92 105.66) (width 0.2) (layer "B.Cu") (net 21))
 (segment (start 134.1 65.54) (end 128.12 65.54) (width 0.2) (layer "F.Cu") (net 16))
 (segment (start 137.885 69.325) (end 134.1 65.54) (width 0.2) (layer "F.Cu") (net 16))
 (segment (start 128.12 65.54) (end 127.62 66.04) (width 0.2) (layer "F.Cu") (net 16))
 (segment (start 137.885 71.865) (end 134.1 68.08) (width 0.2) (layer "F.Cu") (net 15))
 (segment (start 134.1 68.08) (end 128.12 68.08) (width 0.2) (layer "F.Cu") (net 15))
 (segment (start 128.12 68.08) (end 127.62 68.58) (width 0.2) (layer "F.Cu") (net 15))
 (segment (start 177.154 78.096) (end 134.596 78.096) (width 0.2) (layer "F.Cu") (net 18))
 (segment (start 134.596 78.096) (end 127.62 71.12) (width 0.2) (layer "F.Cu") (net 18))
 (segment (start 180.5 74.75) (end 177.154 78.096) (width 0.2) (layer "F.Cu") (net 18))
 (segment (start 180.5 69.75) (end 173.75 63) (width 0.2) (layer "F.Cu") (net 17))
 (segment (start 128.12 63) (end 127.62 63.5) (width 0.2) (layer "F.Cu") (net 17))
 (segment (start 173.75 63) (end 128.12 63) (width 0.2) (layer "F.Cu") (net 17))
 (segment (start 114.5 103) (end 112 105.5) (width 0.2) (layer "F.Cu") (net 3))
 (segment (start 152.332 88.058) (end 145.973586 88.058) (width 0.2) (layer "F.Cu") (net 3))
 (segment (start 145.973586 88.058) (end 131.034586 102.997) (width 0.2) (layer "F.Cu") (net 3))
 (segment (start 131.034586 102.997) (end 123.9359 102.997) (width 0.2) (layer "F.Cu") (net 3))
 (segment (start 123.9359 102.997) (end 123.9329 103) (width 0.2) (layer "F.Cu") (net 3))
 (segment (start 153.07 87.32) (end 152.332 88.058) (width 0.2) (layer "F.Cu") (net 3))
 (segment (start 123.9329 103) (end 114.5 103) (width 0.2) (layer "F.Cu") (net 3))
 (segment (start 139.23874 107.108) (end 135.44874 110.898) (width 0.2) (layer "F.Cu") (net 8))
 (segment (start 113.942 110.898) (end 111.84 113) (width 0.2) (layer "F.Cu") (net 8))
 (segment (start 153.07 106.37) (end 152.332 107.108) (width 0.2) (layer "F.Cu") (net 8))
 (segment (start 135.44874 110.898) (end 113.942 110.898) (width 0.2) (layer "F.Cu") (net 8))
 (segment (start 152.332 107.108) (end 139.23874 107.108) (width 0.2) (layer "F.Cu") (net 8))
 (segment (start 153.07 125.42) (end 152.07 124.42) (width 0.2) (layer "F.Cu") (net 9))
 (segment (start 152.07 124.42) (end 115.76 124.42) (width 0.2) (layer "F.Cu") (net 9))
 (segment (start 115.76 124.42) (end 111.84 120.5) (width 0.2) (layer "F.Cu") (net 9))
 (segment (start 152.489686 107.771) (end 152.227686 107.509) (width 0.2) (layer "F.Cu") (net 6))
 (segment (start 170.981 107.509) (end 153.912314 107.509) (width 0.2) (layer "F.Cu") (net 6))
 (segment (start 153.912314 107.509) (end 153.650314 107.771) (width 0.2) (layer "F.Cu") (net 6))
 (segment (start 152.227686 107.509) (end 139.40484 107.509) (width 0.2) (layer "F.Cu") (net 6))
 (segment (start 135.61484 111.299) (end 123.541 111.299) (width 0.2) (layer "F.Cu") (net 6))
 (segment (start 153.650314 107.771) (end 152.489686 107.771) (width 0.2) (layer "F.Cu") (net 6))
 (segment (start 139.40484 107.509) (end 135.61484 111.299) (width 0.2) (layer "F.Cu") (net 6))
 (segment (start 123.541 111.299) (end 121.84 113) (width 0.2) (layer "F.Cu") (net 6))
 (segment (start 172.12 106.37) (end 170.981 107.509) (width 0.2) (layer "F.Cu") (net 6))
 (segment (start 133.621 103.799) (end 131.92 105.5) (width 0.2) (layer "F.Cu") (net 11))
 (segment (start 190.32847 87.32) (end 173.84947 103.799) (width 0.2) (layer "F.Cu") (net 11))
 (segment (start 173.84947 103.799) (end 133.621 103.799) (width 0.2) (layer "F.Cu") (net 11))
 (segment (start 134.958 123.618) (end 131.84 120.5) (width 0.2) (layer "F.Cu") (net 12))
 (segment (start 191.17 125.42) (end 189.368 123.618) (width 0.2) (layer "F.Cu") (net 12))
 (segment (start 189.368 123.618) (end 134.958 123.618) (width 0.2) (layer "F.Cu") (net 12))
 (segment (start 137.885 74.405) (end 135.9121 74.405) (width 0.2) (layer "F.Cu") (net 14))
 (segment (start 135.9121 74.405) (end 131.1501 69.643) (width 0.2) (layer "F.Cu") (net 14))
 (segment (start 131.1501 69.643) (end 121.063 69.643) (width 0.2) (layer "F.Cu") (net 14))
 (segment (start 121.063 69.643) (end 112.38 60.96) (width 0.2) (layer "F.Cu") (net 14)))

